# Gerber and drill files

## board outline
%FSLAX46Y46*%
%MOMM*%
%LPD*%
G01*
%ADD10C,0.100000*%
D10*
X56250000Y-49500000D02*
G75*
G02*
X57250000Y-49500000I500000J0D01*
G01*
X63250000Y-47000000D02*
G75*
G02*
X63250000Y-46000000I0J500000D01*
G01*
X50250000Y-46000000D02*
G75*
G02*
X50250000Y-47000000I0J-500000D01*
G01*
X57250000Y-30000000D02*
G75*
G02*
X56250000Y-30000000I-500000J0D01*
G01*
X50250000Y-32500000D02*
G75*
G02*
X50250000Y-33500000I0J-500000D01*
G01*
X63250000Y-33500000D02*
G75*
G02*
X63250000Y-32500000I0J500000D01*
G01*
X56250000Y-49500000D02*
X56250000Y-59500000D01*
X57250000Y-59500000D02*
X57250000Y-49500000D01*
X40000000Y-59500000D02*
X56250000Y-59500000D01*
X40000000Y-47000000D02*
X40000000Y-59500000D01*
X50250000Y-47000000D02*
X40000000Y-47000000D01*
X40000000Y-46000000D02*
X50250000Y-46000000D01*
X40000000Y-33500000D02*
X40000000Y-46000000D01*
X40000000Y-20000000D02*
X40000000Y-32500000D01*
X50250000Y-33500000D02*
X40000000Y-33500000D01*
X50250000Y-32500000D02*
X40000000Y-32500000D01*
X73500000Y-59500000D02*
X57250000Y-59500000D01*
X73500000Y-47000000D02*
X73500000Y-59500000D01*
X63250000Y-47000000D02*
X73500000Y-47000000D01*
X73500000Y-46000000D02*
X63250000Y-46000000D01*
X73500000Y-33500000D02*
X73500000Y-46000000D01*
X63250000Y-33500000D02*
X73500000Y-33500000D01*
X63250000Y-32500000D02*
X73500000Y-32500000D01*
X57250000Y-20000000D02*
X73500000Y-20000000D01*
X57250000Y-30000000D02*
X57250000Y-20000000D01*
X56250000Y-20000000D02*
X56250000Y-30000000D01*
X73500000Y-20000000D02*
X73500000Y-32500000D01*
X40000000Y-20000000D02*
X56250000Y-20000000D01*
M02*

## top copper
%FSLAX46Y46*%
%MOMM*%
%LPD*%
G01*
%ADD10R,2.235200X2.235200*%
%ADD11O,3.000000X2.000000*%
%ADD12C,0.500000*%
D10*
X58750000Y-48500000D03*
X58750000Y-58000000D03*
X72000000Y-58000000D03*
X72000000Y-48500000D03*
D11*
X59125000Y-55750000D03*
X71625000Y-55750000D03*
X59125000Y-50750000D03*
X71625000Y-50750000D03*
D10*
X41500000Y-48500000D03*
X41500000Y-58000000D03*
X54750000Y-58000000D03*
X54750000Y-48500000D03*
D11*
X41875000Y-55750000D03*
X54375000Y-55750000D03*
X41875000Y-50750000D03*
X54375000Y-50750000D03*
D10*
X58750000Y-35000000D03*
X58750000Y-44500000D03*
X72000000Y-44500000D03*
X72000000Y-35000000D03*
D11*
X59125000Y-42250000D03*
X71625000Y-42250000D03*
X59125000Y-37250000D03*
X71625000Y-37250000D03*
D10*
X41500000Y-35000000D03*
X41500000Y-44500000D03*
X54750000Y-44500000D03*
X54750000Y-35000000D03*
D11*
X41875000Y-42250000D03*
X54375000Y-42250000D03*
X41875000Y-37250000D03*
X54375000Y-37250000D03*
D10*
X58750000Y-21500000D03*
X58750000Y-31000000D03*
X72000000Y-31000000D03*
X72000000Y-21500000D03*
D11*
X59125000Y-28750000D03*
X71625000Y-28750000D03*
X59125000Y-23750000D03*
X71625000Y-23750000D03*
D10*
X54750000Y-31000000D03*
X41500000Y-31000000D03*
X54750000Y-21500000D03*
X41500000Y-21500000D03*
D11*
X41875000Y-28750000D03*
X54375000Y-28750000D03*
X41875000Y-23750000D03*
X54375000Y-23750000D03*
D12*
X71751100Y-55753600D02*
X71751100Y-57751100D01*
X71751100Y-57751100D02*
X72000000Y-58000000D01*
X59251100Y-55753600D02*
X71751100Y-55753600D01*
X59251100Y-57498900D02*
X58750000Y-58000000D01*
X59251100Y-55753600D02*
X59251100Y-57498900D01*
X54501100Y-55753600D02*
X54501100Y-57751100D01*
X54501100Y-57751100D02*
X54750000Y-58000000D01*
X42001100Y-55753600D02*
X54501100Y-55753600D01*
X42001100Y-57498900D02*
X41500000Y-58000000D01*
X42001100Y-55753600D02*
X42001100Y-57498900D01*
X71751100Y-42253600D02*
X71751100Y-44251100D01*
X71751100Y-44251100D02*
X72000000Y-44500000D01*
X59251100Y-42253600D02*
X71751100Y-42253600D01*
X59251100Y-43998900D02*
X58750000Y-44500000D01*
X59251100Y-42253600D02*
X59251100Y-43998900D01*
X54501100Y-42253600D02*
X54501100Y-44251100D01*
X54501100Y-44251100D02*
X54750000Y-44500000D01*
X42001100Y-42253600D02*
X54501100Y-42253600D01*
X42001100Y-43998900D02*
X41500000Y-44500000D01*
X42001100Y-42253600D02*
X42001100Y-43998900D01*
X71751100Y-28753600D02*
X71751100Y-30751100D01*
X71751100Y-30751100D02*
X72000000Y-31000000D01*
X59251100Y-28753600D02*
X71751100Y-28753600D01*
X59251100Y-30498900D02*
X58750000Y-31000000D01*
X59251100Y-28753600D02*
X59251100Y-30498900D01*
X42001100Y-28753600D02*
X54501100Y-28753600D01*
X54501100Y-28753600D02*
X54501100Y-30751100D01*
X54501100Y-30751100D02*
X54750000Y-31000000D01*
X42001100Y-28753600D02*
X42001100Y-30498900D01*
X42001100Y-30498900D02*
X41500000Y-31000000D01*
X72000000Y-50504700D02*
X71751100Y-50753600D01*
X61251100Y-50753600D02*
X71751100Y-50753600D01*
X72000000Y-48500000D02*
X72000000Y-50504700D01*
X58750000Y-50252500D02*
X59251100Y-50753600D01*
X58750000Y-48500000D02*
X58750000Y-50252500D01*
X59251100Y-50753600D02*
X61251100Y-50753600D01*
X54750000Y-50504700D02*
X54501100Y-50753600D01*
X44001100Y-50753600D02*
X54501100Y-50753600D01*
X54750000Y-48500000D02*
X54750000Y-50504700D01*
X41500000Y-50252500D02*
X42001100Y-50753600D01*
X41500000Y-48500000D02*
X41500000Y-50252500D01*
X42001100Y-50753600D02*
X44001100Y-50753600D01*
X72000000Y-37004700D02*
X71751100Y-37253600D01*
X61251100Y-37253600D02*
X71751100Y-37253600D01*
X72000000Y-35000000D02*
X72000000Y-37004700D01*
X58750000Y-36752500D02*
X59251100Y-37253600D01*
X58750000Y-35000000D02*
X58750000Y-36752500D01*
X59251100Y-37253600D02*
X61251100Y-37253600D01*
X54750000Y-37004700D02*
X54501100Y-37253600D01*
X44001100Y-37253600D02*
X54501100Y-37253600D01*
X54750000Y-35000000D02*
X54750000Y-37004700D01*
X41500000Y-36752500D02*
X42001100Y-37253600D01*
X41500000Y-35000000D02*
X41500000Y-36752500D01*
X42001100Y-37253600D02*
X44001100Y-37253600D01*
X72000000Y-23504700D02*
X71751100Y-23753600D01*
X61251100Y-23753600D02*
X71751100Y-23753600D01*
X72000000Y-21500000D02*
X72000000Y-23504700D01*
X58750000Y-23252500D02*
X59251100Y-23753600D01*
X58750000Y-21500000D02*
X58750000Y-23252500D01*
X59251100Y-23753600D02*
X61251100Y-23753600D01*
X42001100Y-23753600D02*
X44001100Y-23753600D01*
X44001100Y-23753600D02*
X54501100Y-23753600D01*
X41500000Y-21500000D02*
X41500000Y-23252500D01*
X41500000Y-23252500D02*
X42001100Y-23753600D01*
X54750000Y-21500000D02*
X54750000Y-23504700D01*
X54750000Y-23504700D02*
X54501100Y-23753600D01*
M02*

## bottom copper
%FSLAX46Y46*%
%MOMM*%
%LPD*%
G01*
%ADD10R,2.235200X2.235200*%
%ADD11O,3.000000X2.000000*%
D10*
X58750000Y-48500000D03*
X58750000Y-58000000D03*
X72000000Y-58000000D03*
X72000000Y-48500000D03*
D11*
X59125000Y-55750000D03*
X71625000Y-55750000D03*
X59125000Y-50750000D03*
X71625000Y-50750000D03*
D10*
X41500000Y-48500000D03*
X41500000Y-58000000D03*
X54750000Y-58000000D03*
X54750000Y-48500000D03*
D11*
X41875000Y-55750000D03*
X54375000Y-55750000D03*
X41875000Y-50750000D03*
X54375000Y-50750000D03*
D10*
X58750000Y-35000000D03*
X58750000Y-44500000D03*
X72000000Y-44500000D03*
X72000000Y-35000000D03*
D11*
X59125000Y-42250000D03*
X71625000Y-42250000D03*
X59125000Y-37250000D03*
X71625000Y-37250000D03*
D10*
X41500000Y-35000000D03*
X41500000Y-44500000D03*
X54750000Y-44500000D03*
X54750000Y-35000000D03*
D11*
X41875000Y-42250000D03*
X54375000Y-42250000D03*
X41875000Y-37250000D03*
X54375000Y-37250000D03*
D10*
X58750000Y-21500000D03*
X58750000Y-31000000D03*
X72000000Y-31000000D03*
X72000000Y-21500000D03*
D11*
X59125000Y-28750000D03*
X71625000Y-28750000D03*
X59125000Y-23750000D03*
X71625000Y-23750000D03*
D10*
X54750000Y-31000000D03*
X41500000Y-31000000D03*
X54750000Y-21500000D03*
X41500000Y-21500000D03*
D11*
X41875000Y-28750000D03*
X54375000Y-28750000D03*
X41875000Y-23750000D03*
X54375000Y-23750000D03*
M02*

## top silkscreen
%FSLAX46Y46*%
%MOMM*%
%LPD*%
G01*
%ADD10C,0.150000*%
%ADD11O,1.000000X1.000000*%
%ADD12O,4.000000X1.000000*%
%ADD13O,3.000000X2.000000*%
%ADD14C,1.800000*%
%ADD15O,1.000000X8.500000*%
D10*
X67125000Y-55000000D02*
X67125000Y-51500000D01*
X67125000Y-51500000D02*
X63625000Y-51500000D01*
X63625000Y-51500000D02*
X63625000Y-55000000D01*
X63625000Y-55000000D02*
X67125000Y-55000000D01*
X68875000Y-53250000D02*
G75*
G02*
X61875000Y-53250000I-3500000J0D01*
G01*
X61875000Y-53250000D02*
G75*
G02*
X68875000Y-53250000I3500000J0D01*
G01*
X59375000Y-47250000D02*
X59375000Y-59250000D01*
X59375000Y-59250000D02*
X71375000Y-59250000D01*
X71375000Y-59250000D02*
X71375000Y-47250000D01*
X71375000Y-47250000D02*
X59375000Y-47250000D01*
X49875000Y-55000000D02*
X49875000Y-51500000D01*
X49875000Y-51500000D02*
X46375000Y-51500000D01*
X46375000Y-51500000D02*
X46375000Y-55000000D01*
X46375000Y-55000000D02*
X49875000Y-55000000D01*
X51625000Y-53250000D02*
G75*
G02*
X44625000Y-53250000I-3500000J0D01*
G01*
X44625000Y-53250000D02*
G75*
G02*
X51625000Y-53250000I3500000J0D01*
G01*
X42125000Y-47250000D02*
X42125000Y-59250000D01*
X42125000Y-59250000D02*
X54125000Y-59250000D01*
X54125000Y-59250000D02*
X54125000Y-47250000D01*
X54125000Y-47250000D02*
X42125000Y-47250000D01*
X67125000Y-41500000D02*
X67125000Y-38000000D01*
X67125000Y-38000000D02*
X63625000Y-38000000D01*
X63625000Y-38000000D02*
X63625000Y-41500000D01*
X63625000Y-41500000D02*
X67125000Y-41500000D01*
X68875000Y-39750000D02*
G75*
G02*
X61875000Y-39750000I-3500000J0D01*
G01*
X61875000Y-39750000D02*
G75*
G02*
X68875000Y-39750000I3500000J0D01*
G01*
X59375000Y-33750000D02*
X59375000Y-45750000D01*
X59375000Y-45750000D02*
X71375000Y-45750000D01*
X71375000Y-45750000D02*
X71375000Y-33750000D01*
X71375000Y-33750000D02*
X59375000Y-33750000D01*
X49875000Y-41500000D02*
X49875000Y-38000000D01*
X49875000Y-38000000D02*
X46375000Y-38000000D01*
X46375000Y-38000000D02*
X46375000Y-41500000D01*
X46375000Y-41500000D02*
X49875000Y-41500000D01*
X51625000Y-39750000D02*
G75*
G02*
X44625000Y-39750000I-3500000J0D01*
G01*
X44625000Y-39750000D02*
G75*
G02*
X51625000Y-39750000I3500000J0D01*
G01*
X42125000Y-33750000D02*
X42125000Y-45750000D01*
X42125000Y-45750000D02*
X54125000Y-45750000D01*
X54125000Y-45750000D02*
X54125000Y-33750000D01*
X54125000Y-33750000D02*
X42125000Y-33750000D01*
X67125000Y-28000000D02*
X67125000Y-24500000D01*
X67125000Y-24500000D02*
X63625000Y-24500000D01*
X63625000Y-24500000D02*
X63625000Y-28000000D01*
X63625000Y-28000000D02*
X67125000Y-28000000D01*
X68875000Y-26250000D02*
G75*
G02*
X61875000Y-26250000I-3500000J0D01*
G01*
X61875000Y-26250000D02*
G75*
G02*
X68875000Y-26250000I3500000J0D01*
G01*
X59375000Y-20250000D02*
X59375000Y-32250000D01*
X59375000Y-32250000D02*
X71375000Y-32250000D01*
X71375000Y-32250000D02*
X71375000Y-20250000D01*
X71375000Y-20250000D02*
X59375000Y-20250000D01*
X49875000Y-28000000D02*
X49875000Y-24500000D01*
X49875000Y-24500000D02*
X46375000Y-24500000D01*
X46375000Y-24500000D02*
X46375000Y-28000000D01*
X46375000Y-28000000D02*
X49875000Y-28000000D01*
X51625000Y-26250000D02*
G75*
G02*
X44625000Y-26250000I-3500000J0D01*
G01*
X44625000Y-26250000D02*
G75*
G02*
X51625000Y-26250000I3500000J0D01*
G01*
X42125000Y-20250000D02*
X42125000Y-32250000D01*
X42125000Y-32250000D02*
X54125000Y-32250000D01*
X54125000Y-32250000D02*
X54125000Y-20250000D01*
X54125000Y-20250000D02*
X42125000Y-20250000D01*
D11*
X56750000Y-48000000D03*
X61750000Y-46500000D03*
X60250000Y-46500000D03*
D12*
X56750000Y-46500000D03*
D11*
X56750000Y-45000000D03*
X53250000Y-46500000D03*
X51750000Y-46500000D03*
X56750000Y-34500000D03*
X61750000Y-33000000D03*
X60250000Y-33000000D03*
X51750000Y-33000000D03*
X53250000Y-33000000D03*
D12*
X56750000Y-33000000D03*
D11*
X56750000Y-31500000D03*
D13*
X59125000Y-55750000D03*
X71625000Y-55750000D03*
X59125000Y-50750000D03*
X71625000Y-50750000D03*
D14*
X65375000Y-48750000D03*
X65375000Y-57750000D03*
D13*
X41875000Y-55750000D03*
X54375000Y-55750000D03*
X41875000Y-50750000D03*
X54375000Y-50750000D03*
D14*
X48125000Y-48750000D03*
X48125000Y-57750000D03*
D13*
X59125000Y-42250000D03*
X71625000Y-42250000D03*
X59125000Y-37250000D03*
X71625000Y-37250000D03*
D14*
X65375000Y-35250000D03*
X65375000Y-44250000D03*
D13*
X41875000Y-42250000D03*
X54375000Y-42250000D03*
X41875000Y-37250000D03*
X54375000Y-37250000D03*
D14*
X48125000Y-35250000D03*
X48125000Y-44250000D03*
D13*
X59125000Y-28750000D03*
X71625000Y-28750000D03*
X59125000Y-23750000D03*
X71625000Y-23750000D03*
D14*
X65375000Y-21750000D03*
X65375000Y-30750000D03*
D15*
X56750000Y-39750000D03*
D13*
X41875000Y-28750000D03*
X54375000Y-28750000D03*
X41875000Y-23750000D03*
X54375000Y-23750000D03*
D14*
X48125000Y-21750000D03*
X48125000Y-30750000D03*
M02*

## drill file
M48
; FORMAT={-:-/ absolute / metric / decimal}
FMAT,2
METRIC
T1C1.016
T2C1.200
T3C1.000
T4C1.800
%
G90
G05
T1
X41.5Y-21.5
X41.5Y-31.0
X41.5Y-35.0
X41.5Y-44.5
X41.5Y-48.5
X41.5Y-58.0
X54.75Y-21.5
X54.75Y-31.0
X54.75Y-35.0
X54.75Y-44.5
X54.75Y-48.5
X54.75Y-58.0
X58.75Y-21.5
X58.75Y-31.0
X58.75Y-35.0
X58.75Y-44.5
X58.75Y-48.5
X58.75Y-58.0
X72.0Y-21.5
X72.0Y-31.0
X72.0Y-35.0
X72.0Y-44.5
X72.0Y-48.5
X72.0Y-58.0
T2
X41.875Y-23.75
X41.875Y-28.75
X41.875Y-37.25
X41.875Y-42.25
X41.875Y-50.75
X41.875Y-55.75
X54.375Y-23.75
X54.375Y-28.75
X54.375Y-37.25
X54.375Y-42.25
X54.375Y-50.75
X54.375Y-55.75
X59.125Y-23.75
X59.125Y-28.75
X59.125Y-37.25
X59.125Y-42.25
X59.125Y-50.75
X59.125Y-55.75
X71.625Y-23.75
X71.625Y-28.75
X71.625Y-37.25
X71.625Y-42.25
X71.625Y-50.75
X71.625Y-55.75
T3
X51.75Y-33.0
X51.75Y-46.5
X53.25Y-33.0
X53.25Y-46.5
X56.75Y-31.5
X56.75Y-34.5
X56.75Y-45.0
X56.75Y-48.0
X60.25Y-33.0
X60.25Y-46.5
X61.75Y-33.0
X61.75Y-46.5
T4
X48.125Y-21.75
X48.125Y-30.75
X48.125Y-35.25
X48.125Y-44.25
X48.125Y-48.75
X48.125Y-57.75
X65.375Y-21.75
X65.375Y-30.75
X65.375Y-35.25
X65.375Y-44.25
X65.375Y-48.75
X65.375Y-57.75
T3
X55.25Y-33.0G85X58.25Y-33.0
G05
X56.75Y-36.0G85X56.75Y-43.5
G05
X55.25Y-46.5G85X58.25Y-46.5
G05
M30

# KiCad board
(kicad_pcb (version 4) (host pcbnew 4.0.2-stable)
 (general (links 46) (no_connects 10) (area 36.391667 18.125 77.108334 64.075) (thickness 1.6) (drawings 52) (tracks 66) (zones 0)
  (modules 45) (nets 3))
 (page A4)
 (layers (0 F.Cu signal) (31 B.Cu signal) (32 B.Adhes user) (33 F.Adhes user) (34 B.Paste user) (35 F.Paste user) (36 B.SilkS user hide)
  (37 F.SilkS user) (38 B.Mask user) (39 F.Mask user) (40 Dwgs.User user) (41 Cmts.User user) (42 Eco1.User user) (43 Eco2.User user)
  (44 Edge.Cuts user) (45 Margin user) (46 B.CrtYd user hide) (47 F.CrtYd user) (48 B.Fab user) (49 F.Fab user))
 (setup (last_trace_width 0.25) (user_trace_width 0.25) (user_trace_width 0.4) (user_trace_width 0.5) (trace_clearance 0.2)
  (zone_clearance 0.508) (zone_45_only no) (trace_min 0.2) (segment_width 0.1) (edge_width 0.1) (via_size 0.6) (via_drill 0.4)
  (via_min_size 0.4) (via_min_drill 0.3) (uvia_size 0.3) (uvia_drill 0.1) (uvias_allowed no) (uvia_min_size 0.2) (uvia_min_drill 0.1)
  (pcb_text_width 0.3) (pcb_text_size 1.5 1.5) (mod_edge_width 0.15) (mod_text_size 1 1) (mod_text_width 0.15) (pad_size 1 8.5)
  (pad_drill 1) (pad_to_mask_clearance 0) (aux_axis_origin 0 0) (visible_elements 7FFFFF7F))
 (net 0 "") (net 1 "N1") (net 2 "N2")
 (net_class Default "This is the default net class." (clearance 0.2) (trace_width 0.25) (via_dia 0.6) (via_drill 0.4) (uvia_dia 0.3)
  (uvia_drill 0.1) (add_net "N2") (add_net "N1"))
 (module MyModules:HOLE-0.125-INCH (layer F.Cu) (at 56.75 48)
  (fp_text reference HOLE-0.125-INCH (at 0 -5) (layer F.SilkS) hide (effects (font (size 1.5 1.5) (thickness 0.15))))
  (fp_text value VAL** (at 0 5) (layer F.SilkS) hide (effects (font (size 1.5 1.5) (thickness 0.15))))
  (pad "" np_thru_hole oval (at 0 0) (size 1 1) (drill oval 1) (layers *.Cu *.Mask F.SilkS)))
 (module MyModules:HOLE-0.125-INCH (layer F.Cu) (at 61.75 46.5)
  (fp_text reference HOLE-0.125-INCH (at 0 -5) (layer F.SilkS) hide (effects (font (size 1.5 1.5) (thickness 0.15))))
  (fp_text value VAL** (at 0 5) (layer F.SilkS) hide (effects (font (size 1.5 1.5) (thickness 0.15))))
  (pad "" np_thru_hole oval (at 0 0) (size 1 1) (drill oval 1) (layers *.Cu *.Mask F.SilkS)))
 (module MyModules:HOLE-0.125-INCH (layer F.Cu) (at 60.25 46.5)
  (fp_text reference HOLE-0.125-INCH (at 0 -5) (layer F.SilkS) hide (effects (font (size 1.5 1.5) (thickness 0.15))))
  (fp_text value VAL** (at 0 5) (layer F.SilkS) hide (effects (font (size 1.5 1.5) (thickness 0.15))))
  (pad "" np_thru_hole oval (at 0 0) (size 1 1) (drill oval 1) (layers *.Cu *.Mask F.SilkS)))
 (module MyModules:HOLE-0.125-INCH (layer F.Cu) (at 56.75 46.5)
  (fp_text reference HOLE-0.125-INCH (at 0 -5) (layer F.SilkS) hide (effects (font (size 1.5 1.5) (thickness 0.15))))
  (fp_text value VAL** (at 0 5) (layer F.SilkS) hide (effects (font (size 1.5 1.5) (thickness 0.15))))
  (pad "" np_thru_hole oval (at 0 0) (size 4 1) (drill oval 4 1) (layers *.Cu *.Mask F.SilkS)))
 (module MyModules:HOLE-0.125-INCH (layer F.Cu) (at 56.75 45)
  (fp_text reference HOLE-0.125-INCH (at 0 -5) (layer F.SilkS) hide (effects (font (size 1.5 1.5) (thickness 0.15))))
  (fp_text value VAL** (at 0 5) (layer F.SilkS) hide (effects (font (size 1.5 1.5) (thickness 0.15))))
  (pad "" np_thru_hole oval (at 0 0) (size 1 1) (drill oval 1) (layers *.Cu *.Mask F.SilkS)))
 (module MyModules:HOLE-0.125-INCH (layer F.Cu) (at 53.25 46.5)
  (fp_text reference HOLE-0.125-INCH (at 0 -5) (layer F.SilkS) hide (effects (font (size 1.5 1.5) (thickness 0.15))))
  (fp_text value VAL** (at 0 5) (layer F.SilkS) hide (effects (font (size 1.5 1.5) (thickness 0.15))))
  (pad "" np_thru_hole oval (at 0 0) (size 1 1) (drill oval 1) (layers *.Cu *.Mask F.SilkS)))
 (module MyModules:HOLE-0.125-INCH (layer F.Cu) (at 51.75 46.5)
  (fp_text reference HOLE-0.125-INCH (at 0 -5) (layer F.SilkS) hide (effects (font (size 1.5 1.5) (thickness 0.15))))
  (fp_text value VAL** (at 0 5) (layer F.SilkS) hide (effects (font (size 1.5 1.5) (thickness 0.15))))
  (pad "" np_thru_hole oval (at 0 0) (size 1 1) (drill oval 1) (layers *.Cu *.Mask F.SilkS)))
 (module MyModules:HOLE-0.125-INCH (layer F.Cu) (at 56.75 34.5)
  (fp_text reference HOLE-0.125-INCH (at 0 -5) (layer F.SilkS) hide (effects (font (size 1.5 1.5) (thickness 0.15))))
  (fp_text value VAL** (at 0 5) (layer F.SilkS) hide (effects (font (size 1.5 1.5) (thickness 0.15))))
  (pad "" np_thru_hole oval (at 0 0) (size 1 1) (drill oval 1) (layers *.Cu *.Mask F.SilkS)))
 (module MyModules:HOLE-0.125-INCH (layer F.Cu) (at 61.75 33)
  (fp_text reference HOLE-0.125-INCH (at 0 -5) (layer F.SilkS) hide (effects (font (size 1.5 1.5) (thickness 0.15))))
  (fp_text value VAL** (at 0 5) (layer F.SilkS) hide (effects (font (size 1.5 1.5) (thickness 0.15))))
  (pad "" np_thru_hole oval (at 0 0) (size 1 1) (drill oval 1) (layers *.Cu *.Mask F.SilkS)))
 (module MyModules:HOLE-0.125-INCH (layer F.Cu) (at 60.25 33)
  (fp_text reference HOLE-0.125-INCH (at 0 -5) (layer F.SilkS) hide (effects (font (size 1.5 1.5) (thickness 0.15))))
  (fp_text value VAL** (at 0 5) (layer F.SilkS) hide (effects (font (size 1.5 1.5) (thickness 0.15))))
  (pad "" np_thru_hole oval (at 0 0) (size 1 1) (drill oval 1) (layers *.Cu *.Mask F.SilkS)))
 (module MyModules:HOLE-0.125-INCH (layer F.Cu) (at 51.75 33)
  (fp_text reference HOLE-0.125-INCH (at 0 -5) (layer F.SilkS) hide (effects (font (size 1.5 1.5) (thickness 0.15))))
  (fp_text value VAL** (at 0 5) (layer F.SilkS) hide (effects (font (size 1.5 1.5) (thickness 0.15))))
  (pad "" np_thru_hole oval (at 0 0) (size 1 1) (drill oval 1) (layers *.Cu *.Mask F.SilkS)))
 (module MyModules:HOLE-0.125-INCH (layer F.Cu) (at 53.25 33)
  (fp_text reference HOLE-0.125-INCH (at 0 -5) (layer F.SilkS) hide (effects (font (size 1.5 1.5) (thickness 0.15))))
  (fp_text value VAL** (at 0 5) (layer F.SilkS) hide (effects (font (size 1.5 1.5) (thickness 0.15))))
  (pad "" np_thru_hole oval (at 0 0) (size 1 1) (drill oval 1) (layers *.Cu *.Mask F.SilkS)))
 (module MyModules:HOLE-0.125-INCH (layer F.Cu) (at 56.75 33)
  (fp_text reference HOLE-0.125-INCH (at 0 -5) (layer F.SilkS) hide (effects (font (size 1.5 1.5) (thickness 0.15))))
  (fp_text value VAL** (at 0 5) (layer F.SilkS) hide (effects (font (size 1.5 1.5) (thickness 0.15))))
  (pad "" np_thru_hole oval (at 0 0) (size 4 1) (drill oval 4 1) (layers *.Cu *.Mask F.SilkS)))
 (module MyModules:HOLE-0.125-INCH (layer F.Cu) (at 56.75 31.5)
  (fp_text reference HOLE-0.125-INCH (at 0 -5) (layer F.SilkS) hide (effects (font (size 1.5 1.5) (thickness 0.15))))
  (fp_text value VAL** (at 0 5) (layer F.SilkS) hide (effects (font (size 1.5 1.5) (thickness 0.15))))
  (pad "" np_thru_hole oval (at 0 0) (size 1 1) (drill oval 1) (layers *.Cu *.Mask F.SilkS)))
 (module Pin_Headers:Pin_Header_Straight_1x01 (layer B.Cu) (at 58.75 48.5)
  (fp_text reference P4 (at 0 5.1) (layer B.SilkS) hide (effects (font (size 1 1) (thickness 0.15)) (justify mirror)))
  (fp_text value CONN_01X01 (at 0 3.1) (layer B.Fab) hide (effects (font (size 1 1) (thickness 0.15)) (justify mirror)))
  (pad 1 thru_hole rect (at 0 0) (size 2.2352 2.2352) (drill 1.016) (layers *.Cu *.Mask B.SilkS) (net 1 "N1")))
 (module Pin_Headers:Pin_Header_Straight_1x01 (layer B.Cu) (at 58.75 58)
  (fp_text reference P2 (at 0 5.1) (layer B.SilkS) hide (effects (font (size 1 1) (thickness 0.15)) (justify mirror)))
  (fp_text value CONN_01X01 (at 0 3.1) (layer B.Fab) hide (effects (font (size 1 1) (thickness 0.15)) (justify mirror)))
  (pad 1 thru_hole rect (at 0 0) (size 2.2352 2.2352) (drill 1.016) (layers *.Cu *.Mask B.SilkS) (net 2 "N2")))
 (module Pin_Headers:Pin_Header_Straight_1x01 (layer B.Cu) (at 72 58)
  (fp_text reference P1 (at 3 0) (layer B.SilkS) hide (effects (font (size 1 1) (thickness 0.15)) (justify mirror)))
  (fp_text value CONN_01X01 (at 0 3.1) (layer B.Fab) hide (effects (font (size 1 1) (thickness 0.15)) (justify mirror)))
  (pad 1 thru_hole rect (at 0 0) (size 2.2352 2.2352) (drill 1.016) (layers *.Cu *.Mask B.SilkS) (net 2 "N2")))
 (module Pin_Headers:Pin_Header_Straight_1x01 (layer B.Cu) (at 72 48.5)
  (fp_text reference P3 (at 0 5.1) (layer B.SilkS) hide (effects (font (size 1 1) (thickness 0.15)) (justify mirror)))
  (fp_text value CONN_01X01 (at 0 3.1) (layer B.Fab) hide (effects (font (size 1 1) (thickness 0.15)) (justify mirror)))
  (pad 1 thru_hole rect (at 0 0) (size 2.2352 2.2352) (drill 1.016) (layers *.Cu *.Mask B.SilkS) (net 1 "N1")))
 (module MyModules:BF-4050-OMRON (layer F.Cu) (at 65.375 53.25)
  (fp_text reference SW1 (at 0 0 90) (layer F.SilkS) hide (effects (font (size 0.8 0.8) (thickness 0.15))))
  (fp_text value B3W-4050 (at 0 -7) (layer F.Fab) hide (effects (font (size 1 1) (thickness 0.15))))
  (fp_line (start 1.75 1.75) (end 1.75 -1.75) (layer F.SilkS) (width 0.15))
  (fp_line (start 1.75 -1.75) (end -1.75 -1.75) (layer F.SilkS) (width 0.15))
  (fp_line (start -1.75 -1.75) (end -1.75 1.75) (layer F.SilkS) (width 0.15))
  (fp_line (start -1.75 1.75) (end 1.75 1.75) (layer F.SilkS) (width 0.15))
  (fp_circle (center 0 0) (end 3.5 0) (layer F.SilkS) (width 0.15))
  (fp_line (start -6 -6) (end -6 6) (layer F.SilkS) (width 0.15))
  (fp_line (start -6 6) (end 6 6) (layer F.SilkS) (width 0.15))
  (fp_line (start 6 6) (end 6 -6) (layer F.SilkS) (width 0.15))
  (fp_line (start 6 -6) (end -6 -6) (layer F.SilkS) (width 0.15))
  (pad 2 thru_hole oval (at -6.25 2.5) (size 3 2) (drill 1.2) (layers *.Cu *.Mask F.SilkS) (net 2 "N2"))
  (pad 2 thru_hole oval (at 6.25 2.5) (size 3 2) (drill 1.2) (layers *.Cu *.Mask F.SilkS) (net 2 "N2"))
  (pad 1 thru_hole oval (at -6.25 -2.5) (size 3 2) (drill 1.2) (layers *.Cu *.Mask F.SilkS) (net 1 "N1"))
  (pad 1 thru_hole oval (at 6.25 -2.5) (size 3 2) (drill 1.2) (layers *.Cu *.Mask F.SilkS) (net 1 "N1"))
  (pad "" np_thru_hole circle (at 0 -4.5) (size 1.8 1.8) (drill 1.8) (layers *.Cu *.Mask F.SilkS))
  (pad "" np_thru_hole circle (at 0 4.5) (size 1.8 1.8) (drill 1.8) (layers *.Cu *.Mask F.SilkS)))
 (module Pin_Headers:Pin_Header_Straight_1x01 (layer B.Cu) (at 41.5 48.5)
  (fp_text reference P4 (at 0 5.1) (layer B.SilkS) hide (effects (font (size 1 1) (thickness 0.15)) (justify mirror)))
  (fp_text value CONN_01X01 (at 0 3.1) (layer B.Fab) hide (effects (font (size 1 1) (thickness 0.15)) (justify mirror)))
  (pad 1 thru_hole rect (at 0 0) (size 2.2352 2.2352) (drill 1.016) (layers *.Cu *.Mask B.SilkS) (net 1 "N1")))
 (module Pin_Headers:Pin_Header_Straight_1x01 (layer B.Cu) (at 41.5 58)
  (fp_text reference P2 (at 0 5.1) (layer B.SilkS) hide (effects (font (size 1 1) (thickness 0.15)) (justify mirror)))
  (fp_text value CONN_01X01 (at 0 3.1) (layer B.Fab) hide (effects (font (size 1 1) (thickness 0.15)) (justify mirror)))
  (pad 1 thru_hole rect (at 0 0) (size 2.2352 2.2352) (drill 1.016) (layers *.Cu *.Mask B.SilkS) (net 2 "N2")))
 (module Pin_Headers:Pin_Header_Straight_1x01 (layer B.Cu) (at 54.75 58)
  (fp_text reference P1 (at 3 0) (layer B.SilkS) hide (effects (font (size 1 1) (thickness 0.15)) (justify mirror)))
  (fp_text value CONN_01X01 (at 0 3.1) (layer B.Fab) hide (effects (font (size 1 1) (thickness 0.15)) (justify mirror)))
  (pad 1 thru_hole rect (at 0 0) (size 2.2352 2.2352) (drill 1.016) (layers *.Cu *.Mask B.SilkS) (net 2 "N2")))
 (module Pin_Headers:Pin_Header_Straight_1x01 (layer B.Cu) (at 54.75 48.5)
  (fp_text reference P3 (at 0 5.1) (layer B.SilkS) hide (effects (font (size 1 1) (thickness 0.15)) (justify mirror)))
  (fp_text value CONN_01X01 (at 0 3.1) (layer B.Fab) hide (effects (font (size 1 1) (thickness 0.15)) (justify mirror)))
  (pad 1 thru_hole rect (at 0 0) (size 2.2352 2.2352) (drill 1.016) (layers *.Cu *.Mask B.SilkS) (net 1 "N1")))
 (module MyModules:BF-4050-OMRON (layer F.Cu) (at 48.125 53.25)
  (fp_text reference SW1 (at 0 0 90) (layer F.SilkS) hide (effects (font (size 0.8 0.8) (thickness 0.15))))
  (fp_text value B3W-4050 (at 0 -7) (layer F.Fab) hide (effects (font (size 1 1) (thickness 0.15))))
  (fp_line (start 1.75 1.75) (end 1.75 -1.75) (layer F.SilkS) (width 0.15))
  (fp_line (start 1.75 -1.75) (end -1.75 -1.75) (layer F.SilkS) (width 0.15))
  (fp_line (start -1.75 -1.75) (end -1.75 1.75) (layer F.SilkS) (width 0.15))
  (fp_line (start -1.75 1.75) (end 1.75 1.75) (layer F.SilkS) (width 0.15))
  (fp_circle (center 0 0) (end 3.5 0) (layer F.SilkS) (width 0.15))
  (fp_line (start -6 -6) (end -6 6) (layer F.SilkS) (width 0.15))
  (fp_line (start -6 6) (end 6 6) (layer F.SilkS) (width 0.15))
  (fp_line (start 6 6) (end 6 -6) (layer F.SilkS) (width 0.15))
  (fp_line (start 6 -6) (end -6 -6) (layer F.SilkS) (width 0.15))
  (pad 2 thru_hole oval (at -6.25 2.5) (size 3 2) (drill 1.2) (layers *.Cu *.Mask F.SilkS) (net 2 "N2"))
  (pad 2 thru_hole oval (at 6.25 2.5) (size 3 2) (drill 1.2) (layers *.Cu *.Mask F.SilkS) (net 2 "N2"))
  (pad 1 thru_hole oval (at -6.25 -2.5) (size 3 2) (drill 1.2) (layers *.Cu *.Mask F.SilkS) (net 1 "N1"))
  (pad 1 thru_hole oval (at 6.25 -2.5) (size 3 2) (drill 1.2) (layers *.Cu *.Mask F.SilkS) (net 1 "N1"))
  (pad "" np_thru_hole circle (at 0 -4.5) (size 1.8 1.8) (drill 1.8) (layers *.Cu *.Mask F.SilkS))
  (pad "" np_thru_hole circle (at 0 4.5) (size 1.8 1.8) (drill 1.8) (layers *.Cu *.Mask F.SilkS)))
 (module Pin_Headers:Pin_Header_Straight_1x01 (layer B.Cu) (at 58.75 35)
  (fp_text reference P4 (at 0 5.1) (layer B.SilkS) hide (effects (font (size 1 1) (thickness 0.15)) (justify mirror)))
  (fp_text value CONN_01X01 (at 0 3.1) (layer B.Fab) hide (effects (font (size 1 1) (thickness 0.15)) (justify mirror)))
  (pad 1 thru_hole rect (at 0 0) (size 2.2352 2.2352) (drill 1.016) (layers *.Cu *.Mask B.SilkS) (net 1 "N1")))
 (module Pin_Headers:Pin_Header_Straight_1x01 (layer B.Cu) (at 58.75 44.5)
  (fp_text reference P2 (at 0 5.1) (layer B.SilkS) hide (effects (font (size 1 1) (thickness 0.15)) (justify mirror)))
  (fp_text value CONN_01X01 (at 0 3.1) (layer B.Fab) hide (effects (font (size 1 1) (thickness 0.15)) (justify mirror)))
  (pad 1 thru_hole rect (at 0 0) (size 2.2352 2.2352) (drill 1.016) (layers *.Cu *.Mask B.SilkS) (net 2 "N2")))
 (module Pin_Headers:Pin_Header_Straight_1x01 (layer B.Cu) (at 72 44.5)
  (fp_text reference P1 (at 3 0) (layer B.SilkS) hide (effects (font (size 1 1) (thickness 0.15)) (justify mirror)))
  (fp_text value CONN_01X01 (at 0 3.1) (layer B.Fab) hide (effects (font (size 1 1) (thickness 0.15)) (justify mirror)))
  (pad 1 thru_hole rect (at 0 0) (size 2.2352 2.2352) (drill 1.016) (layers *.Cu *.Mask B.SilkS) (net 2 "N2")))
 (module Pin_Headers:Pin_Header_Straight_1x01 (layer B.Cu) (at 72 35)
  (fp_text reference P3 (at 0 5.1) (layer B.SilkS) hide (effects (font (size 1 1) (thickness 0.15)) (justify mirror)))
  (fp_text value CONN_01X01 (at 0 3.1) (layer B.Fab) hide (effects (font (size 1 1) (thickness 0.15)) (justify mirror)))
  (pad 1 thru_hole rect (at 0 0) (size 2.2352 2.2352) (drill 1.016) (layers *.Cu *.Mask B.SilkS) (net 1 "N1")))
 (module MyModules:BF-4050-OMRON (layer F.Cu) (at 65.375 39.75)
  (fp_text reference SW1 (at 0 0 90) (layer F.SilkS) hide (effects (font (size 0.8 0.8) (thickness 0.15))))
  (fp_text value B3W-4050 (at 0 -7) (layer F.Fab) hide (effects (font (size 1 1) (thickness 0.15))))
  (fp_line (start 1.75 1.75) (end 1.75 -1.75) (layer F.SilkS) (width 0.15))
  (fp_line (start 1.75 -1.75) (end -1.75 -1.75) (layer F.SilkS) (width 0.15))
  (fp_line (start -1.75 -1.75) (end -1.75 1.75) (layer F.SilkS) (width 0.15))
  (fp_line (start -1.75 1.75) (end 1.75 1.75) (layer F.SilkS) (width 0.15))
  (fp_circle (center 0 0) (end 3.5 0) (layer F.SilkS) (width 0.15))
  (fp_line (start -6 -6) (end -6 6) (layer F.SilkS) (width 0.15))
  (fp_line (start -6 6) (end 6 6) (layer F.SilkS) (width 0.15))
  (fp_line (start 6 6) (end 6 -6) (layer F.SilkS) (width 0.15))
  (fp_line (start 6 -6) (end -6 -6) (layer F.SilkS) (width 0.15))
  (pad 2 thru_hole oval (at -6.25 2.5) (size 3 2) (drill 1.2) (layers *.Cu *.Mask F.SilkS) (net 2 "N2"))
  (pad 2 thru_hole oval (at 6.25 2.5) (size 3 2) (drill 1.2) (layers *.Cu *.Mask F.SilkS) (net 2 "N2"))
  (pad 1 thru_hole oval (at -6.25 -2.5) (size 3 2) (drill 1.2) (layers *.Cu *.Mask F.SilkS) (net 1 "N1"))
  (pad 1 thru_hole oval (at 6.25 -2.5) (size 3 2) (drill 1.2) (layers *.Cu *.Mask F.SilkS) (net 1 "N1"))
  (pad "" np_thru_hole circle (at 0 -4.5) (size 1.8 1.8) (drill 1.8) (layers *.Cu *.Mask F.SilkS))
  (pad "" np_thru_hole circle (at 0 4.5) (size 1.8 1.8) (drill 1.8) (layers *.Cu *.Mask F.SilkS)))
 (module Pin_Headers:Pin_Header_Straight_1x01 (layer B.Cu) (at 41.5 35)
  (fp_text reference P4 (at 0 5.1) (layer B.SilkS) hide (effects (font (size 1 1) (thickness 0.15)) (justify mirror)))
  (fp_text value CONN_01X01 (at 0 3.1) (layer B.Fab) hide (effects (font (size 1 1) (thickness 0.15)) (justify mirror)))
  (pad 1 thru_hole rect (at 0 0) (size 2.2352 2.2352) (drill 1.016) (layers *.Cu *.Mask B.SilkS) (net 1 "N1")))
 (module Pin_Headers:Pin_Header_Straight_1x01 (layer B.Cu) (at 41.5 44.5)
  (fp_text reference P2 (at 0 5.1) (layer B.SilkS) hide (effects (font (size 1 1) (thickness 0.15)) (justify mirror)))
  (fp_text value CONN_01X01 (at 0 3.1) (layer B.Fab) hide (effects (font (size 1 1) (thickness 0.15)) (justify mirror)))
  (pad 1 thru_hole rect (at 0 0) (size 2.2352 2.2352) (drill 1.016) (layers *.Cu *.Mask B.SilkS) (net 2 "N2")))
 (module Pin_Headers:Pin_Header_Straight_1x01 (layer B.Cu) (at 54.75 44.5)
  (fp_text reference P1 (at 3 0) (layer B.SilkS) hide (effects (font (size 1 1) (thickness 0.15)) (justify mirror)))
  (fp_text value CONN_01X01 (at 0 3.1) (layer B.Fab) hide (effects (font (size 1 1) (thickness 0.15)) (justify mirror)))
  (pad 1 thru_hole rect (at 0 0) (size 2.2352 2.2352) (drill 1.016) (layers *.Cu *.Mask B.SilkS) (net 2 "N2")))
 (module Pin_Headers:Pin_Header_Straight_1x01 (layer B.Cu) (at 54.75 35)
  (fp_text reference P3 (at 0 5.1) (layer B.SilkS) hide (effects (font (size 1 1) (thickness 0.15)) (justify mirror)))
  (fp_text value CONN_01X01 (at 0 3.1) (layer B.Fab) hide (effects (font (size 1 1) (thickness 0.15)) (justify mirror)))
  (pad 1 thru_hole rect (at 0 0) (size 2.2352 2.2352) (drill 1.016) (layers *.Cu *.Mask B.SilkS) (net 1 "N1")))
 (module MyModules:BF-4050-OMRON (layer F.Cu) (at 48.125 39.75)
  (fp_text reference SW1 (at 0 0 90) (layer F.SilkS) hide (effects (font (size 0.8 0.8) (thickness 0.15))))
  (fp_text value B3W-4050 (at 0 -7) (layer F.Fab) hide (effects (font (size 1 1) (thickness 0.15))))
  (fp_line (start 1.75 1.75) (end 1.75 -1.75) (layer F.SilkS) (width 0.15))
  (fp_line (start 1.75 -1.75) (end -1.75 -1.75) (layer F.SilkS) (width 0.15))
  (fp_line (start -1.75 -1.75) (end -1.75 1.75) (layer F.SilkS) (width 0.15))
  (fp_line (start -1.75 1.75) (end 1.75 1.75) (layer F.SilkS) (width 0.15))
  (fp_circle (center 0 0) (end 3.5 0) (layer F.SilkS) (width 0.15))
  (fp_line (start -6 -6) (end -6 6) (layer F.SilkS) (width 0.15))
  (fp_line (start -6 6) (end 6 6) (layer F.SilkS) (width 0.15))
  (fp_line (start 6 6) (end 6 -6) (layer F.SilkS) (width 0.15))
  (fp_line (start 6 -6) (end -6 -6) (layer F.SilkS) (width 0.15))
  (pad 2 thru_hole oval (at -6.25 2.5) (size 3 2) (drill 1.2) (layers *.Cu *.Mask F.SilkS) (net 2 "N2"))
  (pad 2 thru_hole oval (at 6.25 2.5) (size 3 2) (drill 1.2) (layers *.Cu *.Mask F.SilkS) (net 2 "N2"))
  (pad 1 thru_hole oval (at -6.25 -2.5) (size 3 2) (drill 1.2) (layers *.Cu *.Mask F.SilkS) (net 1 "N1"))
  (pad 1 thru_hole oval (at 6.25 -2.5) (size 3 2) (drill 1.2) (layers *.Cu *.Mask F.SilkS) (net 1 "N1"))
  (pad "" np_thru_hole circle (at 0 -4.5) (size 1.8 1.8) (drill 1.8) (layers *.Cu *.Mask F.SilkS))
  (pad "" np_thru_hole circle (at 0 4.5) (size 1.8 1.8) (drill 1.8) (layers *.Cu *.Mask F.SilkS)))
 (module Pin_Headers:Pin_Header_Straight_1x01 (layer B.Cu) (at 58.75 21.5)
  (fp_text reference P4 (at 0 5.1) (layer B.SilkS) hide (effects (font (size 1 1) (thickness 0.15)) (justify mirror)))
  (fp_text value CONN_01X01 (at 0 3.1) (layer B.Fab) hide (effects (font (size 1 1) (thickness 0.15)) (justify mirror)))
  (pad 1 thru_hole rect (at 0 0) (size 2.2352 2.2352) (drill 1.016) (layers *.Cu *.Mask B.SilkS) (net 1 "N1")))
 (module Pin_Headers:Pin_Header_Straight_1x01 (layer B.Cu) (at 58.75 31)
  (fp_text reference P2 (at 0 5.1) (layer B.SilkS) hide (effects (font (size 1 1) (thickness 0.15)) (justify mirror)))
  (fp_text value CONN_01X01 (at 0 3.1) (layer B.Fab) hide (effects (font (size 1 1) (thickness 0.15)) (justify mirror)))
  (pad 1 thru_hole rect (at 0 0) (size 2.2352 2.2352) (drill 1.016) (layers *.Cu *.Mask B.SilkS) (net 2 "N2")))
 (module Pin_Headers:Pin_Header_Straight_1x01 (layer B.Cu) (at 72 31)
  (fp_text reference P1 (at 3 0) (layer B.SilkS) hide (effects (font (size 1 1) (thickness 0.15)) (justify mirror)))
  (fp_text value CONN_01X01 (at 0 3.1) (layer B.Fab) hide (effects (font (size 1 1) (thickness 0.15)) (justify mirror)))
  (pad 1 thru_hole rect (at 0 0) (size 2.2352 2.2352) (drill 1.016) (layers *.Cu *.Mask B.SilkS) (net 2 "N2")))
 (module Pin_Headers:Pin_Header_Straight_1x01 (layer B.Cu) (at 72 21.5)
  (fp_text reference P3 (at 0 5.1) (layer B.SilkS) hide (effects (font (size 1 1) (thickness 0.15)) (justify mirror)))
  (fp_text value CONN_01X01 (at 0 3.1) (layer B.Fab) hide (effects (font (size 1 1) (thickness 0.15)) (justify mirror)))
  (pad 1 thru_hole rect (at 0 0) (size 2.2352 2.2352) (drill 1.016) (layers *.Cu *.Mask B.SilkS) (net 1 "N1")))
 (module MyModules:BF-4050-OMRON (layer F.Cu) (at 65.375 26.25)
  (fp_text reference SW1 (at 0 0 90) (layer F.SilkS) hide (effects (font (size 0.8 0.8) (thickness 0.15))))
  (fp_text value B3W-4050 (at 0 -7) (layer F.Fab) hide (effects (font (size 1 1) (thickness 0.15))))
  (fp_line (start 1.75 1.75) (end 1.75 -1.75) (layer F.SilkS) (width 0.15))
  (fp_line (start 1.75 -1.75) (end -1.75 -1.75) (layer F.SilkS) (width 0.15))
  (fp_line (start -1.75 -1.75) (end -1.75 1.75) (layer F.SilkS) (width 0.15))
  (fp_line (start -1.75 1.75) (end 1.75 1.75) (layer F.SilkS) (width 0.15))
  (fp_circle (center 0 0) (end 3.5 0) (layer F.SilkS) (width 0.15))
  (fp_line (start -6 -6) (end -6 6) (layer F.SilkS) (width 0.15))
  (fp_line (start -6 6) (end 6 6) (layer F.SilkS) (width 0.15))
  (fp_line (start 6 6) (end 6 -6) (layer F.SilkS) (width 0.15))
  (fp_line (start 6 -6) (end -6 -6) (layer F.SilkS) (width 0.15))
  (pad 2 thru_hole oval (at -6.25 2.5) (size 3 2) (drill 1.2) (layers *.Cu *.Mask F.SilkS) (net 2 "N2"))
  (pad 2 thru_hole oval (at 6.25 2.5) (size 3 2) (drill 1.2) (layers *.Cu *.Mask F.SilkS) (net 2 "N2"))
  (pad 1 thru_hole oval (at -6.25 -2.5) (size 3 2) (drill 1.2) (layers *.Cu *.Mask F.SilkS) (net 1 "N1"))
  (pad 1 thru_hole oval (at 6.25 -2.5) (size 3 2) (drill 1.2) (layers *.Cu *.Mask F.SilkS) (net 1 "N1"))
  (pad "" np_thru_hole circle (at 0 -4.5) (size 1.8 1.8) (drill 1.8) (layers *.Cu *.Mask F.SilkS))
  (pad "" np_thru_hole circle (at 0 4.5) (size 1.8 1.8) (drill 1.8) (layers *.Cu *.Mask F.SilkS)))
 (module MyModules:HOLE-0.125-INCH (layer F.Cu) (at 56.75 39.75)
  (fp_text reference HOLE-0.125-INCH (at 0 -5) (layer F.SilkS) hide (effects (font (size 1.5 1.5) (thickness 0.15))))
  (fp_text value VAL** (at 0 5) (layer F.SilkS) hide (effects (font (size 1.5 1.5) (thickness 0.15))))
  (pad "" np_thru_hole oval (at 0 0) (size 1 8.5) (drill oval 1 8.5) (layers *.Cu *.Mask F.SilkS)))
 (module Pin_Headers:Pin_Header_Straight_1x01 (layer B.Cu) (at 54.75 31)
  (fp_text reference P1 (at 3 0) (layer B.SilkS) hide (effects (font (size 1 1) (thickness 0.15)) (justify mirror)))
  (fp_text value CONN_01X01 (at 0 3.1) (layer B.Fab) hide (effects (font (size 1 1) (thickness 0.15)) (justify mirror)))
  (pad 1 thru_hole rect (at 0 0) (size 2.2352 2.2352) (drill 1.016) (layers *.Cu *.Mask B.SilkS) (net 2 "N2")))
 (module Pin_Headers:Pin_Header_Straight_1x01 (layer B.Cu) (at 41.5 31)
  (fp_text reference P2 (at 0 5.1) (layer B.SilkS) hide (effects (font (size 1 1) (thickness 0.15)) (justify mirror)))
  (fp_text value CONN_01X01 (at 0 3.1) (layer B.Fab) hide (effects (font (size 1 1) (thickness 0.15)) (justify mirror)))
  (pad 1 thru_hole rect (at 0 0) (size 2.2352 2.2352) (drill 1.016) (layers *.Cu *.Mask B.SilkS) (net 2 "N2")))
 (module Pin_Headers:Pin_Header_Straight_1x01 (layer B.Cu) (at 54.75 21.5)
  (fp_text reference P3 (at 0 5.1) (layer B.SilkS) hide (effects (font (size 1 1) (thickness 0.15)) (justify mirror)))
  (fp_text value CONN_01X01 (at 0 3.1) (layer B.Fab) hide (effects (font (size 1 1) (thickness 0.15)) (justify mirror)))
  (pad 1 thru_hole rect (at 0 0) (size 2.2352 2.2352) (drill 1.016) (layers *.Cu *.Mask B.SilkS) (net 1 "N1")))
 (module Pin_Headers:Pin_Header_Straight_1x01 (layer B.Cu) (at 41.5 21.5)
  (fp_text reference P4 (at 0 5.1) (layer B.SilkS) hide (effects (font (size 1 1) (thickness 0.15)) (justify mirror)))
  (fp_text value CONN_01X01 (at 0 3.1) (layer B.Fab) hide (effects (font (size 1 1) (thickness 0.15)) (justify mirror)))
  (pad 1 thru_hole rect (at 0 0) (size 2.2352 2.2352) (drill 1.016) (layers *.Cu *.Mask B.SilkS) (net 1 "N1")))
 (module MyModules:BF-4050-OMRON (layer F.Cu) (at 48.125 26.25)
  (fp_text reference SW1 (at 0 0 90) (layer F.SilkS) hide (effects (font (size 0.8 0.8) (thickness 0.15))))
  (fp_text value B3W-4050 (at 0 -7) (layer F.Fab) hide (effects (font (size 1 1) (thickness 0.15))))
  (fp_line (start 1.75 1.75) (end 1.75 -1.75) (layer F.SilkS) (width 0.15))
  (fp_line (start 1.75 -1.75) (end -1.75 -1.75) (layer F.SilkS) (width 0.15))
  (fp_line (start -1.75 -1.75) (end -1.75 1.75) (layer F.SilkS) (width 0.15))
  (fp_line (start -1.75 1.75) (end 1.75 1.75) (layer F.SilkS) (width 0.15))
  (fp_circle (center 0 0) (end 3.5 0) (layer F.SilkS) (width 0.15))
  (fp_line (start -6 -6) (end -6 6) (layer F.SilkS) (width 0.15))
  (fp_line (start -6 6) (end 6 6) (layer F.SilkS) (width 0.15))
  (fp_line (start 6 6) (end 6 -6) (layer F.SilkS) (width 0.15))
  (fp_line (start 6 -6) (end -6 -6) (layer F.SilkS) (width 0.15))
  (pad 2 thru_hole oval (at -6.25 2.5) (size 3 2) (drill 1.2) (layers *.Cu *.Mask F.SilkS) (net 2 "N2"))
  (pad 2 thru_hole oval (at 6.25 2.5) (size 3 2) (drill 1.2) (layers *.Cu *.Mask F.SilkS) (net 2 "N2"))
  (pad 1 thru_hole oval (at -6.25 -2.5) (size 3 2) (drill 1.2) (layers *.Cu *.Mask F.SilkS) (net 1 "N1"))
  (pad 1 thru_hole oval (at 6.25 -2.5) (size 3 2) (drill 1.2) (layers *.Cu *.Mask F.SilkS) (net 1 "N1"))
  (pad "" np_thru_hole circle (at 0 -4.5) (size 1.8 1.8) (drill 1.8) (layers *.Cu *.Mask F.SilkS))
  (pad "" np_thru_hole circle (at 0 4.5) (size 1.8 1.8) (drill 1.8) (layers *.Cu *.Mask F.SilkS)))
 (gr_arc (start 56.75 49.5) (end 56.25 49.5) (angle 180) (layer Edge.Cuts) (width 0.1))
 (gr_arc (start 63.25 46.5) (end 63.25 47) (angle 180) (layer Edge.Cuts) (width 0.1))
 (gr_arc (start 50.25 46.5) (end 50.25 46) (angle 180) (layer Edge.Cuts) (width 0.1))
 (gr_arc (start 56.75 30) (end 57.25 30) (angle 180) (layer Edge.Cuts) (width 0.1))
 (gr_arc (start 50.25 33) (end 50.25 32.5) (angle 180) (layer Edge.Cuts) (width 0.1))
 (gr_arc (start 63.25 33) (end 63.25 33.5) (angle 180) (layer Edge.Cuts) (width 0.1))
 (gr_line (start 56.25 49.5) (end 56.25 59.5) (angle 90) (layer Edge.Cuts) (width 0.1))
 (gr_line (start 57.25 59.5) (end 57.25 49.5) (angle 90) (layer Edge.Cuts) (width 0.1))
 (gr_line (start 40 59.5) (end 56.25 59.5) (layer Edge.Cuts) (width 0.1))
 (gr_line (start 40 47) (end 40 59.5) (layer Edge.Cuts) (width 0.1))
 (gr_line (start 50.25 47) (end 40 47) (layer Edge.Cuts) (width 0.1))
 (gr_line (start 40 46) (end 50.25 46) (layer Edge.Cuts) (width 0.1))
 (gr_line (start 40 33.5) (end 40 46) (layer Edge.Cuts) (width 0.1))
 (gr_line (start 40 20) (end 40 32.5) (layer Edge.Cuts) (width 0.1))
 (gr_line (start 50.25 33.5) (end 40 33.5) (angle 90) (layer Edge.Cuts) (width 0.1))
 (gr_line (start 50.25 32.5) (end 40 32.5) (angle 90) (layer Edge.Cuts) (width 0.1))
 (gr_line (start 73.5 59.5) (end 57.25 59.5) (angle 90) (layer Edge.Cuts) (width 0.1))
 (gr_line (start 73.5 47) (end 73.5 59.5) (angle 90) (layer Edge.Cuts) (width 0.1))
 (gr_line (start 63.25 47) (end 73.5 47) (angle 90) (layer Edge.Cuts) (width 0.1))
 (gr_line (start 73.5 46) (end 63.25 46) (angle 90) (layer Edge.Cuts) (width 0.1))
 (gr_line (start 73.5 33.5) (end 73.5 46) (angle 90) (layer Edge.Cuts) (width 0.1))
 (gr_line (start 63.25 33.5) (end 73.5 33.5) (angle 90) (layer Edge.Cuts) (width 0.1))
 (gr_line (start 63.25 32.5) (end 73.5 32.5) (angle 90) (layer Edge.Cuts) (width 0.1))
 (gr_line (start 57.25 20) (end 73.5 20) (layer Edge.Cuts) (width 0.1))
 (gr_line (start 57.25 30) (end 57.25 20) (layer Edge.Cuts) (width 0.1))
 (gr_line (start 56.25 20) (end 56.25 30) (layer Edge.Cuts) (width 0.1))
 (gr_line (start 73.5 20) (end 73.5 32.5) (layer Edge.Cuts) (width 0.1))
 (gr_line (start 40 20) (end 56.25 20) (layer Edge.Cuts) (width 0.1))
 (segment (start 71.7511 55.7536) (end 71.7511 57.7511) (width 0.5) (layer F.Cu) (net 2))
 (segment (start 71.7511 57.7511) (end 72 58) (width 0.5) (layer F.Cu) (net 2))
 (segment (start 59.2511 55.7536) (end 71.7511 55.7536) (width 0.5) (layer F.Cu) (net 2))
 (segment (start 59.2511 57.4989) (end 58.75 58) (width 0.5) (layer F.Cu) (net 2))
 (segment (start 59.2511 55.7536) (end 59.2511 57.4989) (width 0.5) (layer F.Cu) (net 2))
 (segment (start 54.5011 55.7536) (end 54.5011 57.7511) (width 0.5) (layer F.Cu) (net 2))
 (segment (start 54.5011 57.7511) (end 54.75 58) (width 0.5) (layer F.Cu) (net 2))
 (segment (start 42.0011 55.7536) (end 54.5011 55.7536) (width 0.5) (layer F.Cu) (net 2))
 (segment (start 42.0011 57.4989) (end 41.5 58) (width 0.5) (layer F.Cu) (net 2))
 (segment (start 42.0011 55.7536) (end 42.0011 57.4989) (width 0.5) (layer F.Cu) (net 2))
 (segment (start 71.7511 42.2536) (end 71.7511 44.2511) (width 0.5) (layer F.Cu) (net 2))
 (segment (start 71.7511 44.2511) (end 72 44.5) (width 0.5) (layer F.Cu) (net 2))
 (segment (start 59.2511 42.2536) (end 71.7511 42.2536) (width 0.5) (layer F.Cu) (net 2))
 (segment (start 59.2511 43.9989) (end 58.75 44.5) (width 0.5) (layer F.Cu) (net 2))
 (segment (start 59.2511 42.2536) (end 59.2511 43.9989) (width 0.5) (layer F.Cu) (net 2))
 (segment (start 54.5011 42.2536) (end 54.5011 44.2511) (width 0.5) (layer F.Cu) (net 2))
 (segment (start 54.5011 44.2511) (end 54.75 44.5) (width 0.5) (layer F.Cu) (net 2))
 (segment (start 42.0011 42.2536) (end 54.5011 42.2536) (width 0.5) (layer F.Cu) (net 2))
 (segment (start 42.0011 43.9989) (end 41.5 44.5) (width 0.5) (layer F.Cu) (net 2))
 (segment (start 42.0011 42.2536) (end 42.0011 43.9989) (width 0.5) (layer F.Cu) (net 2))
 (segment (start 71.7511 28.7536) (end 71.7511 30.7511) (width 0.5) (layer F.Cu) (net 2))
 (segment (start 71.7511 30.7511) (end 72 31) (width 0.5) (layer F.Cu) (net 2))
 (segment (start 59.2511 28.7536) (end 71.7511 28.7536) (width 0.5) (layer F.Cu) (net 2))
 (segment (start 59.2511 30.4989) (end 58.75 31) (width 0.5) (layer F.Cu) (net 2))
 (segment (start 59.2511 28.7536) (end 59.2511 30.4989) (width 0.5) (layer F.Cu) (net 2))
 (segment (start 42.0011 28.7536) (end 54.5011 28.7536) (width 0.5) (layer F.Cu) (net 2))
 (segment (start 54.5011 28.7536) (end 54.5011 30.7511) (width 0.5) (layer F.Cu) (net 2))
 (segment (start 54.5011 30.7511) (end 54.75 31) (width 0.5) (layer F.Cu) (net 2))
 (segment (start 42.0011 28.7536) (end 42.0011 30.4989) (width 0.5) (layer F.Cu) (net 2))
 (segment (start 42.0011 30.4989) (end 41.5 31) (width 0.5) (layer F.Cu) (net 2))
 (segment (start 72 50.5047) (end 71.7511 50.7536) (width 0.5) (layer F.Cu) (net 1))
 (segment (start 61.2511 50.7536) (end 71.7511 50.7536) (width 0.5) (layer F.Cu) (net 1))
 (segment (start 72 48.5) (end 72 50.5047) (width 0.5) (layer F.Cu) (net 1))
 (segment (start 58.75 50.2525) (end 59.2511 50.7536) (width 0.5) (layer F.Cu) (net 1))
 (segment (start 58.75 48.5) (end 58.75 50.2525) (width 0.5) (layer F.Cu) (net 1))
 (segment (start 59.2511 50.7536) (end 61.2511 50.7536) (width 0.5) (layer F.Cu) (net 1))
 (segment (start 54.75 50.5047) (end 54.5011 50.7536) (width 0.5) (layer F.Cu) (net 1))
 (segment (start 44.0011 50.7536) (end 54.5011 50.7536) (width 0.5) (layer F.Cu) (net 1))
 (segment (start 54.75 48.5) (end 54.75 50.5047) (width 0.5) (layer F.Cu) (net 1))
 (segment (start 41.5 50.2525) (end 42.0011 50.7536) (width 0.5) (layer F.Cu) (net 1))
 (segment (start 41.5 48.5) (end 41.5 50.2525) (width 0.5) (layer F.Cu) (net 1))
 (segment (start 42.0011 50.7536) (end 44.0011 50.7536) (width 0.5) (layer F.Cu) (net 1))
 (segment (start 72 37.0047) (end 71.7511 37.2536) (width 0.5) (layer F.Cu) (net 1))
 (segment (start 61.2511 37.2536) (end 71.7511 37.2536) (width 0.5) (layer F.Cu) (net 1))
 (segment (start 72 35) (end 72 37.0047) (width 0.5) (layer F.Cu) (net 1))
 (segment (start 58.75 36.7525) (end 59.2511 37.2536) (width 0.5) (layer F.Cu) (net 1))
 (segment (start 58.75 35) (end 58.75 36.7525) (width 0.5) (layer F.Cu) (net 1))
 (segment (start 59.2511 37.2536) (end 61.2511 37.2536) (width 0.5) (layer F.Cu) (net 1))
 (segment (start 54.75 37.0047) (end 54.5011 37.2536) (width 0.5) (layer F.Cu) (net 1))
 (segment (start 44.0011 37.2536) (end 54.5011 37.2536) (width 0.5) (layer F.Cu) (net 1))
 (segment (start 54.75 35) (end 54.75 37.0047) (width 0.5) (layer F.Cu) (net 1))
 (segment (start 41.5 36.7525) (end 42.0011 37.2536) (width 0.5) (layer F.Cu) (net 1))
 (segment (start 41.5 35) (end 41.5 36.7525) (width 0.5) (layer F.Cu) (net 1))
 (segment (start 42.0011 37.2536) (end 44.0011 37.2536) (width 0.5) (layer F.Cu) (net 1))
 (segment (start 72 23.5047) (end 71.7511 23.7536) (width 0.5) (layer F.Cu) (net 1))
 (segment (start 61.2511 23.7536) (end 71.7511 23.7536) (width 0.5) (layer F.Cu) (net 1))
 (segment (start 72 21.5) (end 72 23.5047) (width 0.5) (layer F.Cu) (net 1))
 (segment (start 58.75 23.2525) (end 59.2511 23.7536) (width 0.5) (layer F.Cu) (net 1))
 (segment (start 58.75 21.5) (end 58.75 23.2525) (width 0.5) (layer F.Cu) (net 1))
 (segment (start 59.2511 23.7536) (end 61.2511 23.7536) (width 0.5) (layer F.Cu) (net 1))
 (segment (start 42.0011 23.7536) (end 44.0011 23.7536) (width 0.5) (layer F.Cu) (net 1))
 (segment (start 44.0011 23.7536) (end 54.5011 23.7536) (width 0.5) (layer F.Cu) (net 1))
 (segment (start 41.5 21.5) (end 41.5 23.2525) (width 0.5) (layer F.Cu) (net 1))
 (segment (start 41.5 23.2525) (end 42.0011 23.7536) (width 0.5) (layer F.Cu) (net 1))
 (segment (start 54.75 21.5) (end 54.75 23.5047) (width 0.5) (layer F.Cu) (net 1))
 (segment (start 54.75 23.5047) (end 54.5011 23.7536) (width 0.5) (layer F.Cu) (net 1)))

